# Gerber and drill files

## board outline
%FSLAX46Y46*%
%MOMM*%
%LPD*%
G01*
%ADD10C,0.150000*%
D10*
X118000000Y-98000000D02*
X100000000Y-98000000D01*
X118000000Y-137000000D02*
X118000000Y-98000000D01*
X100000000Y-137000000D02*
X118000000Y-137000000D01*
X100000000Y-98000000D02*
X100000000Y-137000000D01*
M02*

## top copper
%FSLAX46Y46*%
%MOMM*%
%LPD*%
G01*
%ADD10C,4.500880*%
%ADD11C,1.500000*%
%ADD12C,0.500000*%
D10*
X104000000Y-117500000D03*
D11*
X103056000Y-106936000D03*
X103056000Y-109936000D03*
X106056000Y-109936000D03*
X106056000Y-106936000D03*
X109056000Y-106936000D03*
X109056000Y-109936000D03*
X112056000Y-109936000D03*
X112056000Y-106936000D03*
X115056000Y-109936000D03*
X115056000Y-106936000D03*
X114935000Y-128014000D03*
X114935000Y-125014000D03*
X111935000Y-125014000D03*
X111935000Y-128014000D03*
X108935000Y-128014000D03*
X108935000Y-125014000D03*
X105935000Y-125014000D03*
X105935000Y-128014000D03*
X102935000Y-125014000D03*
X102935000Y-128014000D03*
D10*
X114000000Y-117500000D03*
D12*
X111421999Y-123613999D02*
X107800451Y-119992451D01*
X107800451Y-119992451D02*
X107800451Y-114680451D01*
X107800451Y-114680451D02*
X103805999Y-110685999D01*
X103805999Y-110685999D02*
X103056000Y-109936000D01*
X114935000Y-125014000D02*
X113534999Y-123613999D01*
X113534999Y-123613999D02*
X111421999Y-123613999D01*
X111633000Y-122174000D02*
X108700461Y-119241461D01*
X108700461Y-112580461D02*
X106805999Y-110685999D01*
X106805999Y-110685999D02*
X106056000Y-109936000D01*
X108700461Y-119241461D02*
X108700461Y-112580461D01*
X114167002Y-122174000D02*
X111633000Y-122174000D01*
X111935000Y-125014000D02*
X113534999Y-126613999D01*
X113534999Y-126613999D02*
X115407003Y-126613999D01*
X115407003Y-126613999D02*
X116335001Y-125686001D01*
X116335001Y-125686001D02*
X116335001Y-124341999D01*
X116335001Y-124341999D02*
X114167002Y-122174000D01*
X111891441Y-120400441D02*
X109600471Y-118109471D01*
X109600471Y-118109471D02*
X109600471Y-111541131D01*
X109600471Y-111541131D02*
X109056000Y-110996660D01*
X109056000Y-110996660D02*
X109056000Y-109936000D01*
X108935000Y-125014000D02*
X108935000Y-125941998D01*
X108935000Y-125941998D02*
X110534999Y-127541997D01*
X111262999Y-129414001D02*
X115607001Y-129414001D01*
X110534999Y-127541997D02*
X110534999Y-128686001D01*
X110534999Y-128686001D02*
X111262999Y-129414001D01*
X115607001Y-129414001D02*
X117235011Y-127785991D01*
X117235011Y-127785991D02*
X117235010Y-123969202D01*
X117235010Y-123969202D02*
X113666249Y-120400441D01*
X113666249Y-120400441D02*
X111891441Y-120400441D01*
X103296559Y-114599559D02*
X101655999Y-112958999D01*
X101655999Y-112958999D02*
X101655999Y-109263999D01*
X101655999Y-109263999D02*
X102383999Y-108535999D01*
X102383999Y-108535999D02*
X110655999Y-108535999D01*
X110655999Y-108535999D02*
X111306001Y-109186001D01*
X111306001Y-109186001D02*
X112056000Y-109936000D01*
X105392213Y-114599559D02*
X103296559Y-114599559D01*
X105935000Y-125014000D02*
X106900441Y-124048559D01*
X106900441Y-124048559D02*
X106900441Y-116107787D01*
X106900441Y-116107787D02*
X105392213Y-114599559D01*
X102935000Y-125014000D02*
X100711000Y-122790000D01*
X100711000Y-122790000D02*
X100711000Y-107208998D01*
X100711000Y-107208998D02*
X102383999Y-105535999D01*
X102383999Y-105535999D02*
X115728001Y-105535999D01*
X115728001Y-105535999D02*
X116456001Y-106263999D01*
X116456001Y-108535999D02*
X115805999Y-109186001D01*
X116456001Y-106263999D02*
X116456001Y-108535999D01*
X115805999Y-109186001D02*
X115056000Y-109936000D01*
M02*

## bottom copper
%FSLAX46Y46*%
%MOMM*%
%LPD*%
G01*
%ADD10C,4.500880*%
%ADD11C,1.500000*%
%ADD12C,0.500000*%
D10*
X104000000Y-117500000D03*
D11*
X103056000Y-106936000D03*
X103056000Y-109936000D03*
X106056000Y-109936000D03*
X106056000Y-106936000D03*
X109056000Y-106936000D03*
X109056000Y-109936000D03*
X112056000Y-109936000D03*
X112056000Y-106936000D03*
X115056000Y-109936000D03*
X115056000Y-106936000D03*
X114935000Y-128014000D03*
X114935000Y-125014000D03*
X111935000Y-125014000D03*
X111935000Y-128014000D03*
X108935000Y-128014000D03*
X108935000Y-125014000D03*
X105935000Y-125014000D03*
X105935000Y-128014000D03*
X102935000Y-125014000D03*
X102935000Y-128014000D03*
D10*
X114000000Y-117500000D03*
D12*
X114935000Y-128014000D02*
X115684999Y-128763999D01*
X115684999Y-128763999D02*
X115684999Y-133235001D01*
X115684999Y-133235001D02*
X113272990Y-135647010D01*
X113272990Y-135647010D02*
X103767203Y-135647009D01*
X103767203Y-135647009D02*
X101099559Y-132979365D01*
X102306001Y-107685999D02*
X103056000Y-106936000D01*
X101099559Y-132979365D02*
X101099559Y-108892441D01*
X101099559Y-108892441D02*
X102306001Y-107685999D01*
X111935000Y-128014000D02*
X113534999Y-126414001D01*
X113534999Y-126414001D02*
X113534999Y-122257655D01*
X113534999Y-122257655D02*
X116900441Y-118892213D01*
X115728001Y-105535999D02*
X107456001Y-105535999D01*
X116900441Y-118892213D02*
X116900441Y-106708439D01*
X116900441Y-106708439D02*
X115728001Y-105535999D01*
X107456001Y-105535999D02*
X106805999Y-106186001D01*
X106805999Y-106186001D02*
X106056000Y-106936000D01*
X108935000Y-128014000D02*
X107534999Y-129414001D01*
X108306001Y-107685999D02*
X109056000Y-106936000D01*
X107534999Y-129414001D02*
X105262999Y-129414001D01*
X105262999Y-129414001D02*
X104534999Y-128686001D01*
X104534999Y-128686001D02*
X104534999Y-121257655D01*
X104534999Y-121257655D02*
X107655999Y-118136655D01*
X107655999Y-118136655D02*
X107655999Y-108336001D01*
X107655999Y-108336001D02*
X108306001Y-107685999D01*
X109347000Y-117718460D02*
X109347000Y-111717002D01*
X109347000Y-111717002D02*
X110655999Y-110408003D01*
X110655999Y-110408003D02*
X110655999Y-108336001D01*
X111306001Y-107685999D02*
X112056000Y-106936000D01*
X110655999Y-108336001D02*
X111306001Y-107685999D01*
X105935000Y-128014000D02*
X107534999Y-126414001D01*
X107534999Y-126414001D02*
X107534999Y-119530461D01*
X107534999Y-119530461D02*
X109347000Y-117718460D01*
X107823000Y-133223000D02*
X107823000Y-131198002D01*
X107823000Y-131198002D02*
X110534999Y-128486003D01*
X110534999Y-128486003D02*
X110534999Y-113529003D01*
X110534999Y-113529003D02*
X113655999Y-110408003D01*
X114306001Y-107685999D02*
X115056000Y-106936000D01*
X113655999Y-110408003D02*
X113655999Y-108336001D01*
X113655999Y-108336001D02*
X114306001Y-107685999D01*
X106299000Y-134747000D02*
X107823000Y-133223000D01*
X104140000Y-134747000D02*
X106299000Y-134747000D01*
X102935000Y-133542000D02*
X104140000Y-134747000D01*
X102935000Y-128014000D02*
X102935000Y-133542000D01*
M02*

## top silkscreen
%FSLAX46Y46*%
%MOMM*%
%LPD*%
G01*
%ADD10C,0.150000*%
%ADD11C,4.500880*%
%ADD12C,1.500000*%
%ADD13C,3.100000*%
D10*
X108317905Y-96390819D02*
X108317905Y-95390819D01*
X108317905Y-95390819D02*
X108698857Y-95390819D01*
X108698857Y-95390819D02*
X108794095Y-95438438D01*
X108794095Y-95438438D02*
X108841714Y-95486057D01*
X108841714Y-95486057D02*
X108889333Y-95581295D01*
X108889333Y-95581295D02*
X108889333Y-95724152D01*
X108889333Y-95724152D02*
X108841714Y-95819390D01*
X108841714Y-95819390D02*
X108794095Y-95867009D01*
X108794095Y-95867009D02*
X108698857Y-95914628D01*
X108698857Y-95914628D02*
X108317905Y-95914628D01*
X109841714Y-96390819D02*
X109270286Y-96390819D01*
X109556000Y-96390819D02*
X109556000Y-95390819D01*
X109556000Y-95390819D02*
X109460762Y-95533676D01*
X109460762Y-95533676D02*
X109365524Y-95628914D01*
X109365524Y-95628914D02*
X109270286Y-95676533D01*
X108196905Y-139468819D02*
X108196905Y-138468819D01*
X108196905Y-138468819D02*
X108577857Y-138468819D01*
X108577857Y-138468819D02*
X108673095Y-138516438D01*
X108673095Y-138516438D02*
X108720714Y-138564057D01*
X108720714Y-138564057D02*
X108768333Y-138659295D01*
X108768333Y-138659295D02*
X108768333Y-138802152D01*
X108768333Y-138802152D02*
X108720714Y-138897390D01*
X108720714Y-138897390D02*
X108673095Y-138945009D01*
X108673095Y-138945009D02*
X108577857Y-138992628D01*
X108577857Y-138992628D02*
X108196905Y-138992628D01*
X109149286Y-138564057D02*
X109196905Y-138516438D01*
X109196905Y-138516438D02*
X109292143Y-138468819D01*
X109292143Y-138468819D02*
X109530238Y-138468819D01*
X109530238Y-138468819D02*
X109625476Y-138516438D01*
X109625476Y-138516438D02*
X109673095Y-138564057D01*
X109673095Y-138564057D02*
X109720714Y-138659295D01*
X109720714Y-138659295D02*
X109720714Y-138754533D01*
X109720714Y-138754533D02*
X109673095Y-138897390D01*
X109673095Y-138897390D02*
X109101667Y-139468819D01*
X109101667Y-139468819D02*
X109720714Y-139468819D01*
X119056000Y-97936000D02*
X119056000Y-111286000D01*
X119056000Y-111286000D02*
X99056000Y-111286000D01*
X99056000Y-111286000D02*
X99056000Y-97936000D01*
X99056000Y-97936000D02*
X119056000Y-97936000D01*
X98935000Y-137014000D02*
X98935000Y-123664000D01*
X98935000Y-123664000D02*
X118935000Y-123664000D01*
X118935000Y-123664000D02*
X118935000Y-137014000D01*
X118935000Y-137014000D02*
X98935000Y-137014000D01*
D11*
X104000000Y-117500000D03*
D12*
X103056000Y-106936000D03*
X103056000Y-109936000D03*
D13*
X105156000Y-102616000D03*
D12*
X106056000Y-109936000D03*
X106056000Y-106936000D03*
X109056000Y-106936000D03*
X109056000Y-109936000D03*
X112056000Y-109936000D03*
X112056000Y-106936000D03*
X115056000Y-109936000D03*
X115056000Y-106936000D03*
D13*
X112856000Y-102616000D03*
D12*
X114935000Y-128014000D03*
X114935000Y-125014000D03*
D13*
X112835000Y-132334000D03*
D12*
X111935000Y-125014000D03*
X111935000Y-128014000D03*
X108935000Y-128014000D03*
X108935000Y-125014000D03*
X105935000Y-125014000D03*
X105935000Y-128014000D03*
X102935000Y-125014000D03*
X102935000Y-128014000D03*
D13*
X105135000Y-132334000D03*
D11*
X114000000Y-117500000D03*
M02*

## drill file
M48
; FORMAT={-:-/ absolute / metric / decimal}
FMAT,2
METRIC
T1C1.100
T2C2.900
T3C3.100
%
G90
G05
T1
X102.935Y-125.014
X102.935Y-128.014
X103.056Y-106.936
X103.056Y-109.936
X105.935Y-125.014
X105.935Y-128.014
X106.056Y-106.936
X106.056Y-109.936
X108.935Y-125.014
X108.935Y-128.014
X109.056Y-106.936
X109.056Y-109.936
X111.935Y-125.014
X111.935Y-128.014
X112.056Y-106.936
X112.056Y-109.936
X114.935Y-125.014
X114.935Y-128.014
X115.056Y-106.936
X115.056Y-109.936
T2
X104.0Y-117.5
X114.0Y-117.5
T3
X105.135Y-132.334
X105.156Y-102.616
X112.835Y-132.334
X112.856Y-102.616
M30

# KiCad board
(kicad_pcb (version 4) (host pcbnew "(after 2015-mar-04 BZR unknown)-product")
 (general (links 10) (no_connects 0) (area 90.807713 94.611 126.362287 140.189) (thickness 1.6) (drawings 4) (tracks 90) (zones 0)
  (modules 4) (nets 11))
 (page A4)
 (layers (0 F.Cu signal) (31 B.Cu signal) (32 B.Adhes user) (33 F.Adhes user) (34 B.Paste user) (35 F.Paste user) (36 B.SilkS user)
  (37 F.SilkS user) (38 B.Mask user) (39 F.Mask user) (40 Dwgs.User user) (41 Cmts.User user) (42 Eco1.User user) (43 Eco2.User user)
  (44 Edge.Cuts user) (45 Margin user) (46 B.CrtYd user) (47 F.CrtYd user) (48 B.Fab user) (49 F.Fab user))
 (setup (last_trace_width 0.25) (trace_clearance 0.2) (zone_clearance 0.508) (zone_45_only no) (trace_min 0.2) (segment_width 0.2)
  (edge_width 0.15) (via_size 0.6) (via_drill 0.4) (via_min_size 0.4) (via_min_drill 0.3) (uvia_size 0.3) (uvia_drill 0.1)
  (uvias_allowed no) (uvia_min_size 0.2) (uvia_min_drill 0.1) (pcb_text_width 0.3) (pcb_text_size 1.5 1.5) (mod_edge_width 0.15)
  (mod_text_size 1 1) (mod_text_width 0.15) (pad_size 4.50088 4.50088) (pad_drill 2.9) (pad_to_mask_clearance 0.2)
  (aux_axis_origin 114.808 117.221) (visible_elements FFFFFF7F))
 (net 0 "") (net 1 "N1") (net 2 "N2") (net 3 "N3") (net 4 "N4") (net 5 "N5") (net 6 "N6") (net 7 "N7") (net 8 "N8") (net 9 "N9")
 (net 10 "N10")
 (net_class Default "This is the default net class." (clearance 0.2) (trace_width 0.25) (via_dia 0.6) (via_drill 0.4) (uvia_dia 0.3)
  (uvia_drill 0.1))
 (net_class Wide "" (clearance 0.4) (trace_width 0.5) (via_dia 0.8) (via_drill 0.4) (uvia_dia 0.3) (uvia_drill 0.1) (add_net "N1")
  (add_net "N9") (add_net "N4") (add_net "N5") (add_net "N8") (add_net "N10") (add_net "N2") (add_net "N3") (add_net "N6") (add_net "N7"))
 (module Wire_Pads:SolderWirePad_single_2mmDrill (layer F.Cu) (at 103.632 117.221)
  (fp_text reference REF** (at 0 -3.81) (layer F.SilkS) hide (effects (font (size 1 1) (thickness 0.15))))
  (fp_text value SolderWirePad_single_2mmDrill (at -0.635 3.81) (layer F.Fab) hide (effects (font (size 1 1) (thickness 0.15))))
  (pad 1 thru_hole circle (at 0.368 0.279) (size 4.50088 4.50088) (drill 2.9) (layers *.Cu *.Mask F.SilkS)))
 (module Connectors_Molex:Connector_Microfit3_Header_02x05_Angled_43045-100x (layer F.Cu) (at 103.056 106.936 180)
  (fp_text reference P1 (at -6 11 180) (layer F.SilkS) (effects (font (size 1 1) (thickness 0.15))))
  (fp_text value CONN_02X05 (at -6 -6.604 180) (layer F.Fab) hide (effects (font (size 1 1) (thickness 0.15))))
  (fp_line (start -16 9) (end -16 -4.35) (layer F.SilkS) (width 0.15))
  (fp_line (start -16 -4.35) (end 4 -4.35) (layer F.SilkS) (width 0.15))
  (fp_line (start 4 -4.35) (end 4 9) (layer F.SilkS) (width 0.15))
  (fp_line (start 4 9) (end -16 9) (layer F.SilkS) (width 0.15))
  (pad 1 thru_hole circle (at 0 0 180) (size 1.5 1.5) (drill 1.1) (layers *.Cu *.Mask F.SilkS) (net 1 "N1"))
  (pad 6 thru_hole circle (at 0 -3 180) (size 1.5 1.5) (drill 1.1) (layers *.Cu *.Mask F.SilkS) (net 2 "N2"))
  (pad "" np_thru_hole circle (at -2.1 4.32 180) (size 3.1 3.1) (drill 3.1) (layers *.Cu *.Mask F.SilkS))
  (pad 7 thru_hole circle (at -3 -3 180) (size 1.5 1.5) (drill 1.1) (layers *.Cu *.Mask F.SilkS) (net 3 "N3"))
  (pad 2 thru_hole circle (at -3 0 180) (size 1.5 1.5) (drill 1.1) (layers *.Cu *.Mask F.SilkS) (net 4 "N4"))
  (pad 3 thru_hole circle (at -6 0 180) (size 1.5 1.5) (drill 1.1) (layers *.Cu *.Mask F.SilkS) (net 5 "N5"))
  (pad 8 thru_hole circle (at -6 -3 180) (size 1.5 1.5) (drill 1.1) (layers *.Cu *.Mask F.SilkS) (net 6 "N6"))
  (pad 9 thru_hole circle (at -9 -3 180) (size 1.5 1.5) (drill 1.1) (layers *.Cu *.Mask F.SilkS) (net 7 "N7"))
  (pad 4 thru_hole circle (at -9 0 180) (size 1.5 1.5) (drill 1.1) (layers *.Cu *.Mask F.SilkS) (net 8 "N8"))
  (pad 10 thru_hole circle (at -12 -3 180) (size 1.5 1.5) (drill 1.1) (layers *.Cu *.Mask F.SilkS) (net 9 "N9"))
  (pad 5 thru_hole circle (at -12 0 180) (size 1.5 1.5) (drill 1.1) (layers *.Cu *.Mask F.SilkS) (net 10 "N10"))
  (pad "" np_thru_hole circle (at -9.8 4.32 180) (size 3.1 3.1) (drill 3.1) (layers *.Cu *.Mask F.SilkS)))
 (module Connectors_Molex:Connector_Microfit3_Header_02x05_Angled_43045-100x (layer F.Cu) (at 114.935 128.014)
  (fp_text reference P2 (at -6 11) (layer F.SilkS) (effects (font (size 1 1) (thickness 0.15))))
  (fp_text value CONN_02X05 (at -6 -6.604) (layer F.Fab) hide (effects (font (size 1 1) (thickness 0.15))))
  (fp_line (start -16 9) (end -16 -4.35) (layer F.SilkS) (width 0.15))
  (fp_line (start -16 -4.35) (end 4 -4.35) (layer F.SilkS) (width 0.15))
  (fp_line (start 4 -4.35) (end 4 9) (layer F.SilkS) (width 0.15))
  (fp_line (start 4 9) (end -16 9) (layer F.SilkS) (width 0.15))
  (pad 1 thru_hole circle (at 0 0) (size 1.5 1.5) (drill 1.1) (layers *.Cu *.Mask F.SilkS) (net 1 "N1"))
  (pad 6 thru_hole circle (at 0 -3) (size 1.5 1.5) (drill 1.1) (layers *.Cu *.Mask F.SilkS) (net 2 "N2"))
  (pad "" np_thru_hole circle (at -2.1 4.32) (size 3.1 3.1) (drill 3.1) (layers *.Cu *.Mask F.SilkS))
  (pad 7 thru_hole circle (at -3 -3) (size 1.5 1.5) (drill 1.1) (layers *.Cu *.Mask F.SilkS) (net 3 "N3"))
  (pad 2 thru_hole circle (at -3 0) (size 1.5 1.5) (drill 1.1) (layers *.Cu *.Mask F.SilkS) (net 4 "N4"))
  (pad 3 thru_hole circle (at -6 0) (size 1.5 1.5) (drill 1.1) (layers *.Cu *.Mask F.SilkS) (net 5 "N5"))
  (pad 8 thru_hole circle (at -6 -3) (size 1.5 1.5) (drill 1.1) (layers *.Cu *.Mask F.SilkS) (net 6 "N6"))
  (pad 9 thru_hole circle (at -9 -3) (size 1.5 1.5) (drill 1.1) (layers *.Cu *.Mask F.SilkS) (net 7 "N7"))
  (pad 4 thru_hole circle (at -9 0) (size 1.5 1.5) (drill 1.1) (layers *.Cu *.Mask F.SilkS) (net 8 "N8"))
  (pad 10 thru_hole circle (at -12 -3) (size 1.5 1.5) (drill 1.1) (layers *.Cu *.Mask F.SilkS) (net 9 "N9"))
  (pad 5 thru_hole circle (at -12 0) (size 1.5 1.5) (drill 1.1) (layers *.Cu *.Mask F.SilkS) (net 10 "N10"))
  (pad "" np_thru_hole circle (at -9.8 4.32) (size 3.1 3.1) (drill 3.1) (layers *.Cu *.Mask F.SilkS)))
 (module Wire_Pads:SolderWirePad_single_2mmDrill (layer F.Cu) (at 114.808 117.348)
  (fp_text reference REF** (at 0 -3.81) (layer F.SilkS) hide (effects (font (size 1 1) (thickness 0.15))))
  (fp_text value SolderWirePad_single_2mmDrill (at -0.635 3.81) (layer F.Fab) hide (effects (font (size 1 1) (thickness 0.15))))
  (pad 1 thru_hole circle (at -0.808 0.152) (size 4.50088 4.50088) (drill 2.9) (layers *.Cu *.Mask F.SilkS)))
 (gr_line (start 118 98) (end 100 98) (angle 90) (layer Edge.Cuts) (width 0.15))
 (gr_line (start 118 137) (end 118 98) (angle 90) (layer Edge.Cuts) (width 0.15))
 (gr_line (start 100 137) (end 118 137) (angle 90) (layer Edge.Cuts) (width 0.15))
 (gr_line (start 100 98) (end 100 137) (angle 90) (layer Edge.Cuts) (width 0.15))
 (segment (start 114.935 128.014) (end 115.684999 128.763999) (width 0.5) (layer B.Cu) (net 1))
 (segment (start 115.684999 128.763999) (end 115.684999 133.235001) (width 0.5) (layer B.Cu) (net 1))
 (segment (start 115.684999 133.235001) (end 113.27299 135.64701) (width 0.5) (layer B.Cu) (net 1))
 (segment (start 113.27299 135.64701) (end 103.767203 135.647009) (width 0.5) (layer B.Cu) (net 1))
 (segment (start 103.767203 135.647009) (end 101.099559 132.979365) (width 0.5) (layer B.Cu) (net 1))
 (segment (start 102.306001 107.685999) (end 103.056 106.936) (width 0.5) (layer B.Cu) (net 1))
 (segment (start 101.099559 132.979365) (end 101.099559 108.892441) (width 0.5) (layer B.Cu) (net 1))
 (segment (start 101.099559 108.892441) (end 102.306001 107.685999) (width 0.5) (layer B.Cu) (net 1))
 (segment (start 111.421999 123.613999) (end 107.800451 119.992451) (width 0.5) (layer F.Cu) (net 2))
 (segment (start 107.800451 119.992451) (end 107.800451 114.680451) (width 0.5) (layer F.Cu) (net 2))
 (segment (start 107.800451 114.680451) (end 103.805999 110.685999) (width 0.5) (layer F.Cu) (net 2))
 (segment (start 103.805999 110.685999) (end 103.056 109.936) (width 0.5) (layer F.Cu) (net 2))
 (segment (start 114.935 125.014) (end 113.534999 123.613999) (width 0.5) (layer F.Cu) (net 2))
 (segment (start 113.534999 123.613999) (end 111.421999 123.613999) (width 0.5) (layer F.Cu) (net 2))
 (segment (start 111.633 122.174) (end 108.700461 119.241461) (width 0.5) (layer F.Cu) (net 3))
 (segment (start 108.700461 112.580461) (end 106.805999 110.685999) (width 0.5) (layer F.Cu) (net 3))
 (segment (start 106.805999 110.685999) (end 106.056 109.936) (width 0.5) (layer F.Cu) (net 3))
 (segment (start 108.700461 119.241461) (end 108.700461 112.580461) (width 0.5) (layer F.Cu) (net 3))
 (segment (start 114.167002 122.174) (end 111.633 122.174) (width 0.5) (layer F.Cu) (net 3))
 (segment (start 111.935 125.014) (end 113.534999 126.613999) (width 0.5) (layer F.Cu) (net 3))
 (segment (start 113.534999 126.613999) (end 115.407003 126.613999) (width 0.5) (layer F.Cu) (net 3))
 (segment (start 115.407003 126.613999) (end 116.335001 125.686001) (width 0.5) (layer F.Cu) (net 3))
 (segment (start 116.335001 125.686001) (end 116.335001 124.341999) (width 0.5) (layer F.Cu) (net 3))
 (segment (start 116.335001 124.341999) (end 114.167002 122.174) (width 0.5) (layer F.Cu) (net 3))
 (segment (start 111.935 128.014) (end 113.534999 126.414001) (width 0.5) (layer B.Cu) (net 4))
 (segment (start 113.534999 126.414001) (end 113.534999 122.257655) (width 0.5) (layer B.Cu) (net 4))
 (segment (start 113.534999 122.257655) (end 116.900441 118.892213) (width 0.5) (layer B.Cu) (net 4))
 (segment (start 115.728001 105.535999) (end 107.456001 105.535999) (width 0.5) (layer B.Cu) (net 4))
 (segment (start 116.900441 118.892213) (end 116.900441 106.708439) (width 0.5) (layer B.Cu) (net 4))
 (segment (start 116.900441 106.708439) (end 115.728001 105.535999) (width 0.5) (layer B.Cu) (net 4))
 (segment (start 107.456001 105.535999) (end 106.805999 106.186001) (width 0.5) (layer B.Cu) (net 4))
 (segment (start 106.805999 106.186001) (end 106.056 106.936) (width 0.5) (layer B.Cu) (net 4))
 (segment (start 108.935 128.014) (end 107.534999 129.414001) (width 0.5) (layer B.Cu) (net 5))
 (segment (start 108.306001 107.685999) (end 109.056 106.936) (width 0.5) (layer B.Cu) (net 5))
 (segment (start 107.534999 129.414001) (end 105.262999 129.414001) (width 0.5) (layer B.Cu) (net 5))
 (segment (start 105.262999 129.414001) (end 104.534999 128.686001) (width 0.5) (layer B.Cu) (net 5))
 (segment (start 104.534999 128.686001) (end 104.534999 121.257655) (width 0.5) (layer B.Cu) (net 5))
 (segment (start 104.534999 121.257655) (end 107.655999 118.136655) (width 0.5) (layer B.Cu) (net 5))
 (segment (start 107.655999 118.136655) (end 107.655999 108.336001) (width 0.5) (layer B.Cu) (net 5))
 (segment (start 107.655999 108.336001) (end 108.306001 107.685999) (width 0.5) (layer B.Cu) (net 5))
 (segment (start 111.891441 120.400441) (end 109.600471 118.109471) (width 0.5) (layer F.Cu) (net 6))
 (segment (start 109.600471 118.109471) (end 109.600471 111.541131) (width 0.5) (layer F.Cu) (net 6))
 (segment (start 109.600471 111.541131) (end 109.056 110.99666) (width 0.5) (layer F.Cu) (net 6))
 (segment (start 109.056 110.99666) (end 109.056 109.936) (width 0.5) (layer F.Cu) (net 6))
 (segment (start 108.935 125.014) (end 108.935 125.941998) (width 0.5) (layer F.Cu) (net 6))
 (segment (start 108.935 125.941998) (end 110.534999 127.541997) (width 0.5) (layer F.Cu) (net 6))
 (segment (start 111.262999 129.414001) (end 115.607001 129.414001) (width 0.5) (layer F.Cu) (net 6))
 (segment (start 110.534999 127.541997) (end 110.534999 128.686001) (width 0.5) (layer F.Cu) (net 6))
 (segment (start 110.534999 128.686001) (end 111.262999 129.414001) (width 0.5) (layer F.Cu) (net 6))
 (segment (start 115.607001 129.414001) (end 117.235011 127.785991) (width 0.5) (layer F.Cu) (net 6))
 (segment (start 117.235011 127.785991) (end 117.23501 123.969202) (width 0.5) (layer F.Cu) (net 6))
 (segment (start 117.23501 123.969202) (end 113.666249 120.400441) (width 0.5) (layer F.Cu) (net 6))
 (segment (start 113.666249 120.400441) (end 111.891441 120.400441) (width 0.5) (layer F.Cu) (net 6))
 (segment (start 103.296559 114.599559) (end 101.655999 112.958999) (width 0.5) (layer F.Cu) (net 7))
 (segment (start 101.655999 112.958999) (end 101.655999 109.263999) (width 0.5) (layer F.Cu) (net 7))
 (segment (start 101.655999 109.263999) (end 102.383999 108.535999) (width 0.5) (layer F.Cu) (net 7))
 (segment (start 102.383999 108.535999) (end 110.655999 108.535999) (width 0.5) (layer F.Cu) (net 7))
 (segment (start 110.655999 108.535999) (end 111.306001 109.186001) (width 0.5) (layer F.Cu) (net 7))
 (segment (start 111.306001 109.186001) (end 112.056 109.936) (width 0.5) (layer F.Cu) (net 7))
 (segment (start 105.392213 114.599559) (end 103.296559 114.599559) (width 0.5) (layer F.Cu) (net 7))
 (segment (start 105.935 125.014) (end 106.900441 124.048559) (width 0.5) (layer F.Cu) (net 7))
 (segment (start 106.900441 124.048559) (end 106.900441 116.107787) (width 0.5) (layer F.Cu) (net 7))
 (segment (start 106.900441 116.107787) (end 105.392213 114.599559) (width 0.5) (layer F.Cu) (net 7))
 (segment (start 109.347 117.71846) (end 109.347 111.717002) (width 0.5) (layer B.Cu) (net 8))
 (segment (start 109.347 111.717002) (end 110.655999 110.408003) (width 0.5) (layer B.Cu) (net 8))
 (segment (start 110.655999 110.408003) (end 110.655999 108.336001) (width 0.5) (layer B.Cu) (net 8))
 (segment (start 111.306001 107.685999) (end 112.056 106.936) (width 0.5) (layer B.Cu) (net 8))
 (segment (start 110.655999 108.336001) (end 111.306001 107.685999) (width 0.5) (layer B.Cu) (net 8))
 (segment (start 105.935 128.014) (end 107.534999 126.414001) (width 0.5) (layer B.Cu) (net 8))
 (segment (start 107.534999 126.414001) (end 107.534999 119.530461) (width 0.5) (layer B.Cu) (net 8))
 (segment (start 107.534999 119.530461) (end 109.347 117.71846) (width 0.5) (layer B.Cu) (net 8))
 (segment (start 102.935 125.014) (end 100.711 122.79) (width 0.5) (layer F.Cu) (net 9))
 (segment (start 100.711 122.79) (end 100.711 107.208998) (width 0.5) (layer F.Cu) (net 9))
 (segment (start 100.711 107.208998) (end 102.383999 105.535999) (width 0.5) (layer F.Cu) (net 9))
 (segment (start 102.383999 105.535999) (end 115.728001 105.535999) (width 0.5) (layer F.Cu) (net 9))
 (segment (start 115.728001 105.535999) (end 116.456001 106.263999) (width 0.5) (layer F.Cu) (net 9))
 (segment (start 116.456001 108.535999) (end 115.805999 109.186001) (width 0.5) (layer F.Cu) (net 9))
 (segment (start 116.456001 106.263999) (end 116.456001 108.535999) (width 0.5) (layer F.Cu) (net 9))
 (segment (start 115.805999 109.186001) (end 115.056 109.936) (width 0.5) (layer F.Cu) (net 9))
 (segment (start 107.823 133.223) (end 107.823 131.198002) (width 0.5) (layer B.Cu) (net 10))
 (segment (start 107.823 131.198002) (end 110.534999 128.486003) (width 0.5) (layer B.Cu) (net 10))
 (segment (start 110.534999 128.486003) (end 110.534999 113.529003) (width 0.5) (layer B.Cu) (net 10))
 (segment (start 110.534999 113.529003) (end 113.655999 110.408003) (width 0.5) (layer B.Cu) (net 10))
 (segment (start 114.306001 107.685999) (end 115.056 106.936) (width 0.5) (layer B.Cu) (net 10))
 (segment (start 113.655999 110.408003) (end 113.655999 108.336001) (width 0.5) (layer B.Cu) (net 10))
 (segment (start 113.655999 108.336001) (end 114.306001 107.685999) (width 0.5) (layer B.Cu) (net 10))
 (segment (start 106.299 134.747) (end 107.823 133.223) (width 0.5) (layer B.Cu) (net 10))
 (segment (start 104.14 134.747) (end 106.299 134.747) (width 0.5) (layer B.Cu) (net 10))
 (segment (start 102.935 133.542) (end 104.14 134.747) (width 0.5) (layer B.Cu) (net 10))
 (segment (start 102.935 128.014) (end 102.935 133.542) (width 0.5) (layer B.Cu) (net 10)))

